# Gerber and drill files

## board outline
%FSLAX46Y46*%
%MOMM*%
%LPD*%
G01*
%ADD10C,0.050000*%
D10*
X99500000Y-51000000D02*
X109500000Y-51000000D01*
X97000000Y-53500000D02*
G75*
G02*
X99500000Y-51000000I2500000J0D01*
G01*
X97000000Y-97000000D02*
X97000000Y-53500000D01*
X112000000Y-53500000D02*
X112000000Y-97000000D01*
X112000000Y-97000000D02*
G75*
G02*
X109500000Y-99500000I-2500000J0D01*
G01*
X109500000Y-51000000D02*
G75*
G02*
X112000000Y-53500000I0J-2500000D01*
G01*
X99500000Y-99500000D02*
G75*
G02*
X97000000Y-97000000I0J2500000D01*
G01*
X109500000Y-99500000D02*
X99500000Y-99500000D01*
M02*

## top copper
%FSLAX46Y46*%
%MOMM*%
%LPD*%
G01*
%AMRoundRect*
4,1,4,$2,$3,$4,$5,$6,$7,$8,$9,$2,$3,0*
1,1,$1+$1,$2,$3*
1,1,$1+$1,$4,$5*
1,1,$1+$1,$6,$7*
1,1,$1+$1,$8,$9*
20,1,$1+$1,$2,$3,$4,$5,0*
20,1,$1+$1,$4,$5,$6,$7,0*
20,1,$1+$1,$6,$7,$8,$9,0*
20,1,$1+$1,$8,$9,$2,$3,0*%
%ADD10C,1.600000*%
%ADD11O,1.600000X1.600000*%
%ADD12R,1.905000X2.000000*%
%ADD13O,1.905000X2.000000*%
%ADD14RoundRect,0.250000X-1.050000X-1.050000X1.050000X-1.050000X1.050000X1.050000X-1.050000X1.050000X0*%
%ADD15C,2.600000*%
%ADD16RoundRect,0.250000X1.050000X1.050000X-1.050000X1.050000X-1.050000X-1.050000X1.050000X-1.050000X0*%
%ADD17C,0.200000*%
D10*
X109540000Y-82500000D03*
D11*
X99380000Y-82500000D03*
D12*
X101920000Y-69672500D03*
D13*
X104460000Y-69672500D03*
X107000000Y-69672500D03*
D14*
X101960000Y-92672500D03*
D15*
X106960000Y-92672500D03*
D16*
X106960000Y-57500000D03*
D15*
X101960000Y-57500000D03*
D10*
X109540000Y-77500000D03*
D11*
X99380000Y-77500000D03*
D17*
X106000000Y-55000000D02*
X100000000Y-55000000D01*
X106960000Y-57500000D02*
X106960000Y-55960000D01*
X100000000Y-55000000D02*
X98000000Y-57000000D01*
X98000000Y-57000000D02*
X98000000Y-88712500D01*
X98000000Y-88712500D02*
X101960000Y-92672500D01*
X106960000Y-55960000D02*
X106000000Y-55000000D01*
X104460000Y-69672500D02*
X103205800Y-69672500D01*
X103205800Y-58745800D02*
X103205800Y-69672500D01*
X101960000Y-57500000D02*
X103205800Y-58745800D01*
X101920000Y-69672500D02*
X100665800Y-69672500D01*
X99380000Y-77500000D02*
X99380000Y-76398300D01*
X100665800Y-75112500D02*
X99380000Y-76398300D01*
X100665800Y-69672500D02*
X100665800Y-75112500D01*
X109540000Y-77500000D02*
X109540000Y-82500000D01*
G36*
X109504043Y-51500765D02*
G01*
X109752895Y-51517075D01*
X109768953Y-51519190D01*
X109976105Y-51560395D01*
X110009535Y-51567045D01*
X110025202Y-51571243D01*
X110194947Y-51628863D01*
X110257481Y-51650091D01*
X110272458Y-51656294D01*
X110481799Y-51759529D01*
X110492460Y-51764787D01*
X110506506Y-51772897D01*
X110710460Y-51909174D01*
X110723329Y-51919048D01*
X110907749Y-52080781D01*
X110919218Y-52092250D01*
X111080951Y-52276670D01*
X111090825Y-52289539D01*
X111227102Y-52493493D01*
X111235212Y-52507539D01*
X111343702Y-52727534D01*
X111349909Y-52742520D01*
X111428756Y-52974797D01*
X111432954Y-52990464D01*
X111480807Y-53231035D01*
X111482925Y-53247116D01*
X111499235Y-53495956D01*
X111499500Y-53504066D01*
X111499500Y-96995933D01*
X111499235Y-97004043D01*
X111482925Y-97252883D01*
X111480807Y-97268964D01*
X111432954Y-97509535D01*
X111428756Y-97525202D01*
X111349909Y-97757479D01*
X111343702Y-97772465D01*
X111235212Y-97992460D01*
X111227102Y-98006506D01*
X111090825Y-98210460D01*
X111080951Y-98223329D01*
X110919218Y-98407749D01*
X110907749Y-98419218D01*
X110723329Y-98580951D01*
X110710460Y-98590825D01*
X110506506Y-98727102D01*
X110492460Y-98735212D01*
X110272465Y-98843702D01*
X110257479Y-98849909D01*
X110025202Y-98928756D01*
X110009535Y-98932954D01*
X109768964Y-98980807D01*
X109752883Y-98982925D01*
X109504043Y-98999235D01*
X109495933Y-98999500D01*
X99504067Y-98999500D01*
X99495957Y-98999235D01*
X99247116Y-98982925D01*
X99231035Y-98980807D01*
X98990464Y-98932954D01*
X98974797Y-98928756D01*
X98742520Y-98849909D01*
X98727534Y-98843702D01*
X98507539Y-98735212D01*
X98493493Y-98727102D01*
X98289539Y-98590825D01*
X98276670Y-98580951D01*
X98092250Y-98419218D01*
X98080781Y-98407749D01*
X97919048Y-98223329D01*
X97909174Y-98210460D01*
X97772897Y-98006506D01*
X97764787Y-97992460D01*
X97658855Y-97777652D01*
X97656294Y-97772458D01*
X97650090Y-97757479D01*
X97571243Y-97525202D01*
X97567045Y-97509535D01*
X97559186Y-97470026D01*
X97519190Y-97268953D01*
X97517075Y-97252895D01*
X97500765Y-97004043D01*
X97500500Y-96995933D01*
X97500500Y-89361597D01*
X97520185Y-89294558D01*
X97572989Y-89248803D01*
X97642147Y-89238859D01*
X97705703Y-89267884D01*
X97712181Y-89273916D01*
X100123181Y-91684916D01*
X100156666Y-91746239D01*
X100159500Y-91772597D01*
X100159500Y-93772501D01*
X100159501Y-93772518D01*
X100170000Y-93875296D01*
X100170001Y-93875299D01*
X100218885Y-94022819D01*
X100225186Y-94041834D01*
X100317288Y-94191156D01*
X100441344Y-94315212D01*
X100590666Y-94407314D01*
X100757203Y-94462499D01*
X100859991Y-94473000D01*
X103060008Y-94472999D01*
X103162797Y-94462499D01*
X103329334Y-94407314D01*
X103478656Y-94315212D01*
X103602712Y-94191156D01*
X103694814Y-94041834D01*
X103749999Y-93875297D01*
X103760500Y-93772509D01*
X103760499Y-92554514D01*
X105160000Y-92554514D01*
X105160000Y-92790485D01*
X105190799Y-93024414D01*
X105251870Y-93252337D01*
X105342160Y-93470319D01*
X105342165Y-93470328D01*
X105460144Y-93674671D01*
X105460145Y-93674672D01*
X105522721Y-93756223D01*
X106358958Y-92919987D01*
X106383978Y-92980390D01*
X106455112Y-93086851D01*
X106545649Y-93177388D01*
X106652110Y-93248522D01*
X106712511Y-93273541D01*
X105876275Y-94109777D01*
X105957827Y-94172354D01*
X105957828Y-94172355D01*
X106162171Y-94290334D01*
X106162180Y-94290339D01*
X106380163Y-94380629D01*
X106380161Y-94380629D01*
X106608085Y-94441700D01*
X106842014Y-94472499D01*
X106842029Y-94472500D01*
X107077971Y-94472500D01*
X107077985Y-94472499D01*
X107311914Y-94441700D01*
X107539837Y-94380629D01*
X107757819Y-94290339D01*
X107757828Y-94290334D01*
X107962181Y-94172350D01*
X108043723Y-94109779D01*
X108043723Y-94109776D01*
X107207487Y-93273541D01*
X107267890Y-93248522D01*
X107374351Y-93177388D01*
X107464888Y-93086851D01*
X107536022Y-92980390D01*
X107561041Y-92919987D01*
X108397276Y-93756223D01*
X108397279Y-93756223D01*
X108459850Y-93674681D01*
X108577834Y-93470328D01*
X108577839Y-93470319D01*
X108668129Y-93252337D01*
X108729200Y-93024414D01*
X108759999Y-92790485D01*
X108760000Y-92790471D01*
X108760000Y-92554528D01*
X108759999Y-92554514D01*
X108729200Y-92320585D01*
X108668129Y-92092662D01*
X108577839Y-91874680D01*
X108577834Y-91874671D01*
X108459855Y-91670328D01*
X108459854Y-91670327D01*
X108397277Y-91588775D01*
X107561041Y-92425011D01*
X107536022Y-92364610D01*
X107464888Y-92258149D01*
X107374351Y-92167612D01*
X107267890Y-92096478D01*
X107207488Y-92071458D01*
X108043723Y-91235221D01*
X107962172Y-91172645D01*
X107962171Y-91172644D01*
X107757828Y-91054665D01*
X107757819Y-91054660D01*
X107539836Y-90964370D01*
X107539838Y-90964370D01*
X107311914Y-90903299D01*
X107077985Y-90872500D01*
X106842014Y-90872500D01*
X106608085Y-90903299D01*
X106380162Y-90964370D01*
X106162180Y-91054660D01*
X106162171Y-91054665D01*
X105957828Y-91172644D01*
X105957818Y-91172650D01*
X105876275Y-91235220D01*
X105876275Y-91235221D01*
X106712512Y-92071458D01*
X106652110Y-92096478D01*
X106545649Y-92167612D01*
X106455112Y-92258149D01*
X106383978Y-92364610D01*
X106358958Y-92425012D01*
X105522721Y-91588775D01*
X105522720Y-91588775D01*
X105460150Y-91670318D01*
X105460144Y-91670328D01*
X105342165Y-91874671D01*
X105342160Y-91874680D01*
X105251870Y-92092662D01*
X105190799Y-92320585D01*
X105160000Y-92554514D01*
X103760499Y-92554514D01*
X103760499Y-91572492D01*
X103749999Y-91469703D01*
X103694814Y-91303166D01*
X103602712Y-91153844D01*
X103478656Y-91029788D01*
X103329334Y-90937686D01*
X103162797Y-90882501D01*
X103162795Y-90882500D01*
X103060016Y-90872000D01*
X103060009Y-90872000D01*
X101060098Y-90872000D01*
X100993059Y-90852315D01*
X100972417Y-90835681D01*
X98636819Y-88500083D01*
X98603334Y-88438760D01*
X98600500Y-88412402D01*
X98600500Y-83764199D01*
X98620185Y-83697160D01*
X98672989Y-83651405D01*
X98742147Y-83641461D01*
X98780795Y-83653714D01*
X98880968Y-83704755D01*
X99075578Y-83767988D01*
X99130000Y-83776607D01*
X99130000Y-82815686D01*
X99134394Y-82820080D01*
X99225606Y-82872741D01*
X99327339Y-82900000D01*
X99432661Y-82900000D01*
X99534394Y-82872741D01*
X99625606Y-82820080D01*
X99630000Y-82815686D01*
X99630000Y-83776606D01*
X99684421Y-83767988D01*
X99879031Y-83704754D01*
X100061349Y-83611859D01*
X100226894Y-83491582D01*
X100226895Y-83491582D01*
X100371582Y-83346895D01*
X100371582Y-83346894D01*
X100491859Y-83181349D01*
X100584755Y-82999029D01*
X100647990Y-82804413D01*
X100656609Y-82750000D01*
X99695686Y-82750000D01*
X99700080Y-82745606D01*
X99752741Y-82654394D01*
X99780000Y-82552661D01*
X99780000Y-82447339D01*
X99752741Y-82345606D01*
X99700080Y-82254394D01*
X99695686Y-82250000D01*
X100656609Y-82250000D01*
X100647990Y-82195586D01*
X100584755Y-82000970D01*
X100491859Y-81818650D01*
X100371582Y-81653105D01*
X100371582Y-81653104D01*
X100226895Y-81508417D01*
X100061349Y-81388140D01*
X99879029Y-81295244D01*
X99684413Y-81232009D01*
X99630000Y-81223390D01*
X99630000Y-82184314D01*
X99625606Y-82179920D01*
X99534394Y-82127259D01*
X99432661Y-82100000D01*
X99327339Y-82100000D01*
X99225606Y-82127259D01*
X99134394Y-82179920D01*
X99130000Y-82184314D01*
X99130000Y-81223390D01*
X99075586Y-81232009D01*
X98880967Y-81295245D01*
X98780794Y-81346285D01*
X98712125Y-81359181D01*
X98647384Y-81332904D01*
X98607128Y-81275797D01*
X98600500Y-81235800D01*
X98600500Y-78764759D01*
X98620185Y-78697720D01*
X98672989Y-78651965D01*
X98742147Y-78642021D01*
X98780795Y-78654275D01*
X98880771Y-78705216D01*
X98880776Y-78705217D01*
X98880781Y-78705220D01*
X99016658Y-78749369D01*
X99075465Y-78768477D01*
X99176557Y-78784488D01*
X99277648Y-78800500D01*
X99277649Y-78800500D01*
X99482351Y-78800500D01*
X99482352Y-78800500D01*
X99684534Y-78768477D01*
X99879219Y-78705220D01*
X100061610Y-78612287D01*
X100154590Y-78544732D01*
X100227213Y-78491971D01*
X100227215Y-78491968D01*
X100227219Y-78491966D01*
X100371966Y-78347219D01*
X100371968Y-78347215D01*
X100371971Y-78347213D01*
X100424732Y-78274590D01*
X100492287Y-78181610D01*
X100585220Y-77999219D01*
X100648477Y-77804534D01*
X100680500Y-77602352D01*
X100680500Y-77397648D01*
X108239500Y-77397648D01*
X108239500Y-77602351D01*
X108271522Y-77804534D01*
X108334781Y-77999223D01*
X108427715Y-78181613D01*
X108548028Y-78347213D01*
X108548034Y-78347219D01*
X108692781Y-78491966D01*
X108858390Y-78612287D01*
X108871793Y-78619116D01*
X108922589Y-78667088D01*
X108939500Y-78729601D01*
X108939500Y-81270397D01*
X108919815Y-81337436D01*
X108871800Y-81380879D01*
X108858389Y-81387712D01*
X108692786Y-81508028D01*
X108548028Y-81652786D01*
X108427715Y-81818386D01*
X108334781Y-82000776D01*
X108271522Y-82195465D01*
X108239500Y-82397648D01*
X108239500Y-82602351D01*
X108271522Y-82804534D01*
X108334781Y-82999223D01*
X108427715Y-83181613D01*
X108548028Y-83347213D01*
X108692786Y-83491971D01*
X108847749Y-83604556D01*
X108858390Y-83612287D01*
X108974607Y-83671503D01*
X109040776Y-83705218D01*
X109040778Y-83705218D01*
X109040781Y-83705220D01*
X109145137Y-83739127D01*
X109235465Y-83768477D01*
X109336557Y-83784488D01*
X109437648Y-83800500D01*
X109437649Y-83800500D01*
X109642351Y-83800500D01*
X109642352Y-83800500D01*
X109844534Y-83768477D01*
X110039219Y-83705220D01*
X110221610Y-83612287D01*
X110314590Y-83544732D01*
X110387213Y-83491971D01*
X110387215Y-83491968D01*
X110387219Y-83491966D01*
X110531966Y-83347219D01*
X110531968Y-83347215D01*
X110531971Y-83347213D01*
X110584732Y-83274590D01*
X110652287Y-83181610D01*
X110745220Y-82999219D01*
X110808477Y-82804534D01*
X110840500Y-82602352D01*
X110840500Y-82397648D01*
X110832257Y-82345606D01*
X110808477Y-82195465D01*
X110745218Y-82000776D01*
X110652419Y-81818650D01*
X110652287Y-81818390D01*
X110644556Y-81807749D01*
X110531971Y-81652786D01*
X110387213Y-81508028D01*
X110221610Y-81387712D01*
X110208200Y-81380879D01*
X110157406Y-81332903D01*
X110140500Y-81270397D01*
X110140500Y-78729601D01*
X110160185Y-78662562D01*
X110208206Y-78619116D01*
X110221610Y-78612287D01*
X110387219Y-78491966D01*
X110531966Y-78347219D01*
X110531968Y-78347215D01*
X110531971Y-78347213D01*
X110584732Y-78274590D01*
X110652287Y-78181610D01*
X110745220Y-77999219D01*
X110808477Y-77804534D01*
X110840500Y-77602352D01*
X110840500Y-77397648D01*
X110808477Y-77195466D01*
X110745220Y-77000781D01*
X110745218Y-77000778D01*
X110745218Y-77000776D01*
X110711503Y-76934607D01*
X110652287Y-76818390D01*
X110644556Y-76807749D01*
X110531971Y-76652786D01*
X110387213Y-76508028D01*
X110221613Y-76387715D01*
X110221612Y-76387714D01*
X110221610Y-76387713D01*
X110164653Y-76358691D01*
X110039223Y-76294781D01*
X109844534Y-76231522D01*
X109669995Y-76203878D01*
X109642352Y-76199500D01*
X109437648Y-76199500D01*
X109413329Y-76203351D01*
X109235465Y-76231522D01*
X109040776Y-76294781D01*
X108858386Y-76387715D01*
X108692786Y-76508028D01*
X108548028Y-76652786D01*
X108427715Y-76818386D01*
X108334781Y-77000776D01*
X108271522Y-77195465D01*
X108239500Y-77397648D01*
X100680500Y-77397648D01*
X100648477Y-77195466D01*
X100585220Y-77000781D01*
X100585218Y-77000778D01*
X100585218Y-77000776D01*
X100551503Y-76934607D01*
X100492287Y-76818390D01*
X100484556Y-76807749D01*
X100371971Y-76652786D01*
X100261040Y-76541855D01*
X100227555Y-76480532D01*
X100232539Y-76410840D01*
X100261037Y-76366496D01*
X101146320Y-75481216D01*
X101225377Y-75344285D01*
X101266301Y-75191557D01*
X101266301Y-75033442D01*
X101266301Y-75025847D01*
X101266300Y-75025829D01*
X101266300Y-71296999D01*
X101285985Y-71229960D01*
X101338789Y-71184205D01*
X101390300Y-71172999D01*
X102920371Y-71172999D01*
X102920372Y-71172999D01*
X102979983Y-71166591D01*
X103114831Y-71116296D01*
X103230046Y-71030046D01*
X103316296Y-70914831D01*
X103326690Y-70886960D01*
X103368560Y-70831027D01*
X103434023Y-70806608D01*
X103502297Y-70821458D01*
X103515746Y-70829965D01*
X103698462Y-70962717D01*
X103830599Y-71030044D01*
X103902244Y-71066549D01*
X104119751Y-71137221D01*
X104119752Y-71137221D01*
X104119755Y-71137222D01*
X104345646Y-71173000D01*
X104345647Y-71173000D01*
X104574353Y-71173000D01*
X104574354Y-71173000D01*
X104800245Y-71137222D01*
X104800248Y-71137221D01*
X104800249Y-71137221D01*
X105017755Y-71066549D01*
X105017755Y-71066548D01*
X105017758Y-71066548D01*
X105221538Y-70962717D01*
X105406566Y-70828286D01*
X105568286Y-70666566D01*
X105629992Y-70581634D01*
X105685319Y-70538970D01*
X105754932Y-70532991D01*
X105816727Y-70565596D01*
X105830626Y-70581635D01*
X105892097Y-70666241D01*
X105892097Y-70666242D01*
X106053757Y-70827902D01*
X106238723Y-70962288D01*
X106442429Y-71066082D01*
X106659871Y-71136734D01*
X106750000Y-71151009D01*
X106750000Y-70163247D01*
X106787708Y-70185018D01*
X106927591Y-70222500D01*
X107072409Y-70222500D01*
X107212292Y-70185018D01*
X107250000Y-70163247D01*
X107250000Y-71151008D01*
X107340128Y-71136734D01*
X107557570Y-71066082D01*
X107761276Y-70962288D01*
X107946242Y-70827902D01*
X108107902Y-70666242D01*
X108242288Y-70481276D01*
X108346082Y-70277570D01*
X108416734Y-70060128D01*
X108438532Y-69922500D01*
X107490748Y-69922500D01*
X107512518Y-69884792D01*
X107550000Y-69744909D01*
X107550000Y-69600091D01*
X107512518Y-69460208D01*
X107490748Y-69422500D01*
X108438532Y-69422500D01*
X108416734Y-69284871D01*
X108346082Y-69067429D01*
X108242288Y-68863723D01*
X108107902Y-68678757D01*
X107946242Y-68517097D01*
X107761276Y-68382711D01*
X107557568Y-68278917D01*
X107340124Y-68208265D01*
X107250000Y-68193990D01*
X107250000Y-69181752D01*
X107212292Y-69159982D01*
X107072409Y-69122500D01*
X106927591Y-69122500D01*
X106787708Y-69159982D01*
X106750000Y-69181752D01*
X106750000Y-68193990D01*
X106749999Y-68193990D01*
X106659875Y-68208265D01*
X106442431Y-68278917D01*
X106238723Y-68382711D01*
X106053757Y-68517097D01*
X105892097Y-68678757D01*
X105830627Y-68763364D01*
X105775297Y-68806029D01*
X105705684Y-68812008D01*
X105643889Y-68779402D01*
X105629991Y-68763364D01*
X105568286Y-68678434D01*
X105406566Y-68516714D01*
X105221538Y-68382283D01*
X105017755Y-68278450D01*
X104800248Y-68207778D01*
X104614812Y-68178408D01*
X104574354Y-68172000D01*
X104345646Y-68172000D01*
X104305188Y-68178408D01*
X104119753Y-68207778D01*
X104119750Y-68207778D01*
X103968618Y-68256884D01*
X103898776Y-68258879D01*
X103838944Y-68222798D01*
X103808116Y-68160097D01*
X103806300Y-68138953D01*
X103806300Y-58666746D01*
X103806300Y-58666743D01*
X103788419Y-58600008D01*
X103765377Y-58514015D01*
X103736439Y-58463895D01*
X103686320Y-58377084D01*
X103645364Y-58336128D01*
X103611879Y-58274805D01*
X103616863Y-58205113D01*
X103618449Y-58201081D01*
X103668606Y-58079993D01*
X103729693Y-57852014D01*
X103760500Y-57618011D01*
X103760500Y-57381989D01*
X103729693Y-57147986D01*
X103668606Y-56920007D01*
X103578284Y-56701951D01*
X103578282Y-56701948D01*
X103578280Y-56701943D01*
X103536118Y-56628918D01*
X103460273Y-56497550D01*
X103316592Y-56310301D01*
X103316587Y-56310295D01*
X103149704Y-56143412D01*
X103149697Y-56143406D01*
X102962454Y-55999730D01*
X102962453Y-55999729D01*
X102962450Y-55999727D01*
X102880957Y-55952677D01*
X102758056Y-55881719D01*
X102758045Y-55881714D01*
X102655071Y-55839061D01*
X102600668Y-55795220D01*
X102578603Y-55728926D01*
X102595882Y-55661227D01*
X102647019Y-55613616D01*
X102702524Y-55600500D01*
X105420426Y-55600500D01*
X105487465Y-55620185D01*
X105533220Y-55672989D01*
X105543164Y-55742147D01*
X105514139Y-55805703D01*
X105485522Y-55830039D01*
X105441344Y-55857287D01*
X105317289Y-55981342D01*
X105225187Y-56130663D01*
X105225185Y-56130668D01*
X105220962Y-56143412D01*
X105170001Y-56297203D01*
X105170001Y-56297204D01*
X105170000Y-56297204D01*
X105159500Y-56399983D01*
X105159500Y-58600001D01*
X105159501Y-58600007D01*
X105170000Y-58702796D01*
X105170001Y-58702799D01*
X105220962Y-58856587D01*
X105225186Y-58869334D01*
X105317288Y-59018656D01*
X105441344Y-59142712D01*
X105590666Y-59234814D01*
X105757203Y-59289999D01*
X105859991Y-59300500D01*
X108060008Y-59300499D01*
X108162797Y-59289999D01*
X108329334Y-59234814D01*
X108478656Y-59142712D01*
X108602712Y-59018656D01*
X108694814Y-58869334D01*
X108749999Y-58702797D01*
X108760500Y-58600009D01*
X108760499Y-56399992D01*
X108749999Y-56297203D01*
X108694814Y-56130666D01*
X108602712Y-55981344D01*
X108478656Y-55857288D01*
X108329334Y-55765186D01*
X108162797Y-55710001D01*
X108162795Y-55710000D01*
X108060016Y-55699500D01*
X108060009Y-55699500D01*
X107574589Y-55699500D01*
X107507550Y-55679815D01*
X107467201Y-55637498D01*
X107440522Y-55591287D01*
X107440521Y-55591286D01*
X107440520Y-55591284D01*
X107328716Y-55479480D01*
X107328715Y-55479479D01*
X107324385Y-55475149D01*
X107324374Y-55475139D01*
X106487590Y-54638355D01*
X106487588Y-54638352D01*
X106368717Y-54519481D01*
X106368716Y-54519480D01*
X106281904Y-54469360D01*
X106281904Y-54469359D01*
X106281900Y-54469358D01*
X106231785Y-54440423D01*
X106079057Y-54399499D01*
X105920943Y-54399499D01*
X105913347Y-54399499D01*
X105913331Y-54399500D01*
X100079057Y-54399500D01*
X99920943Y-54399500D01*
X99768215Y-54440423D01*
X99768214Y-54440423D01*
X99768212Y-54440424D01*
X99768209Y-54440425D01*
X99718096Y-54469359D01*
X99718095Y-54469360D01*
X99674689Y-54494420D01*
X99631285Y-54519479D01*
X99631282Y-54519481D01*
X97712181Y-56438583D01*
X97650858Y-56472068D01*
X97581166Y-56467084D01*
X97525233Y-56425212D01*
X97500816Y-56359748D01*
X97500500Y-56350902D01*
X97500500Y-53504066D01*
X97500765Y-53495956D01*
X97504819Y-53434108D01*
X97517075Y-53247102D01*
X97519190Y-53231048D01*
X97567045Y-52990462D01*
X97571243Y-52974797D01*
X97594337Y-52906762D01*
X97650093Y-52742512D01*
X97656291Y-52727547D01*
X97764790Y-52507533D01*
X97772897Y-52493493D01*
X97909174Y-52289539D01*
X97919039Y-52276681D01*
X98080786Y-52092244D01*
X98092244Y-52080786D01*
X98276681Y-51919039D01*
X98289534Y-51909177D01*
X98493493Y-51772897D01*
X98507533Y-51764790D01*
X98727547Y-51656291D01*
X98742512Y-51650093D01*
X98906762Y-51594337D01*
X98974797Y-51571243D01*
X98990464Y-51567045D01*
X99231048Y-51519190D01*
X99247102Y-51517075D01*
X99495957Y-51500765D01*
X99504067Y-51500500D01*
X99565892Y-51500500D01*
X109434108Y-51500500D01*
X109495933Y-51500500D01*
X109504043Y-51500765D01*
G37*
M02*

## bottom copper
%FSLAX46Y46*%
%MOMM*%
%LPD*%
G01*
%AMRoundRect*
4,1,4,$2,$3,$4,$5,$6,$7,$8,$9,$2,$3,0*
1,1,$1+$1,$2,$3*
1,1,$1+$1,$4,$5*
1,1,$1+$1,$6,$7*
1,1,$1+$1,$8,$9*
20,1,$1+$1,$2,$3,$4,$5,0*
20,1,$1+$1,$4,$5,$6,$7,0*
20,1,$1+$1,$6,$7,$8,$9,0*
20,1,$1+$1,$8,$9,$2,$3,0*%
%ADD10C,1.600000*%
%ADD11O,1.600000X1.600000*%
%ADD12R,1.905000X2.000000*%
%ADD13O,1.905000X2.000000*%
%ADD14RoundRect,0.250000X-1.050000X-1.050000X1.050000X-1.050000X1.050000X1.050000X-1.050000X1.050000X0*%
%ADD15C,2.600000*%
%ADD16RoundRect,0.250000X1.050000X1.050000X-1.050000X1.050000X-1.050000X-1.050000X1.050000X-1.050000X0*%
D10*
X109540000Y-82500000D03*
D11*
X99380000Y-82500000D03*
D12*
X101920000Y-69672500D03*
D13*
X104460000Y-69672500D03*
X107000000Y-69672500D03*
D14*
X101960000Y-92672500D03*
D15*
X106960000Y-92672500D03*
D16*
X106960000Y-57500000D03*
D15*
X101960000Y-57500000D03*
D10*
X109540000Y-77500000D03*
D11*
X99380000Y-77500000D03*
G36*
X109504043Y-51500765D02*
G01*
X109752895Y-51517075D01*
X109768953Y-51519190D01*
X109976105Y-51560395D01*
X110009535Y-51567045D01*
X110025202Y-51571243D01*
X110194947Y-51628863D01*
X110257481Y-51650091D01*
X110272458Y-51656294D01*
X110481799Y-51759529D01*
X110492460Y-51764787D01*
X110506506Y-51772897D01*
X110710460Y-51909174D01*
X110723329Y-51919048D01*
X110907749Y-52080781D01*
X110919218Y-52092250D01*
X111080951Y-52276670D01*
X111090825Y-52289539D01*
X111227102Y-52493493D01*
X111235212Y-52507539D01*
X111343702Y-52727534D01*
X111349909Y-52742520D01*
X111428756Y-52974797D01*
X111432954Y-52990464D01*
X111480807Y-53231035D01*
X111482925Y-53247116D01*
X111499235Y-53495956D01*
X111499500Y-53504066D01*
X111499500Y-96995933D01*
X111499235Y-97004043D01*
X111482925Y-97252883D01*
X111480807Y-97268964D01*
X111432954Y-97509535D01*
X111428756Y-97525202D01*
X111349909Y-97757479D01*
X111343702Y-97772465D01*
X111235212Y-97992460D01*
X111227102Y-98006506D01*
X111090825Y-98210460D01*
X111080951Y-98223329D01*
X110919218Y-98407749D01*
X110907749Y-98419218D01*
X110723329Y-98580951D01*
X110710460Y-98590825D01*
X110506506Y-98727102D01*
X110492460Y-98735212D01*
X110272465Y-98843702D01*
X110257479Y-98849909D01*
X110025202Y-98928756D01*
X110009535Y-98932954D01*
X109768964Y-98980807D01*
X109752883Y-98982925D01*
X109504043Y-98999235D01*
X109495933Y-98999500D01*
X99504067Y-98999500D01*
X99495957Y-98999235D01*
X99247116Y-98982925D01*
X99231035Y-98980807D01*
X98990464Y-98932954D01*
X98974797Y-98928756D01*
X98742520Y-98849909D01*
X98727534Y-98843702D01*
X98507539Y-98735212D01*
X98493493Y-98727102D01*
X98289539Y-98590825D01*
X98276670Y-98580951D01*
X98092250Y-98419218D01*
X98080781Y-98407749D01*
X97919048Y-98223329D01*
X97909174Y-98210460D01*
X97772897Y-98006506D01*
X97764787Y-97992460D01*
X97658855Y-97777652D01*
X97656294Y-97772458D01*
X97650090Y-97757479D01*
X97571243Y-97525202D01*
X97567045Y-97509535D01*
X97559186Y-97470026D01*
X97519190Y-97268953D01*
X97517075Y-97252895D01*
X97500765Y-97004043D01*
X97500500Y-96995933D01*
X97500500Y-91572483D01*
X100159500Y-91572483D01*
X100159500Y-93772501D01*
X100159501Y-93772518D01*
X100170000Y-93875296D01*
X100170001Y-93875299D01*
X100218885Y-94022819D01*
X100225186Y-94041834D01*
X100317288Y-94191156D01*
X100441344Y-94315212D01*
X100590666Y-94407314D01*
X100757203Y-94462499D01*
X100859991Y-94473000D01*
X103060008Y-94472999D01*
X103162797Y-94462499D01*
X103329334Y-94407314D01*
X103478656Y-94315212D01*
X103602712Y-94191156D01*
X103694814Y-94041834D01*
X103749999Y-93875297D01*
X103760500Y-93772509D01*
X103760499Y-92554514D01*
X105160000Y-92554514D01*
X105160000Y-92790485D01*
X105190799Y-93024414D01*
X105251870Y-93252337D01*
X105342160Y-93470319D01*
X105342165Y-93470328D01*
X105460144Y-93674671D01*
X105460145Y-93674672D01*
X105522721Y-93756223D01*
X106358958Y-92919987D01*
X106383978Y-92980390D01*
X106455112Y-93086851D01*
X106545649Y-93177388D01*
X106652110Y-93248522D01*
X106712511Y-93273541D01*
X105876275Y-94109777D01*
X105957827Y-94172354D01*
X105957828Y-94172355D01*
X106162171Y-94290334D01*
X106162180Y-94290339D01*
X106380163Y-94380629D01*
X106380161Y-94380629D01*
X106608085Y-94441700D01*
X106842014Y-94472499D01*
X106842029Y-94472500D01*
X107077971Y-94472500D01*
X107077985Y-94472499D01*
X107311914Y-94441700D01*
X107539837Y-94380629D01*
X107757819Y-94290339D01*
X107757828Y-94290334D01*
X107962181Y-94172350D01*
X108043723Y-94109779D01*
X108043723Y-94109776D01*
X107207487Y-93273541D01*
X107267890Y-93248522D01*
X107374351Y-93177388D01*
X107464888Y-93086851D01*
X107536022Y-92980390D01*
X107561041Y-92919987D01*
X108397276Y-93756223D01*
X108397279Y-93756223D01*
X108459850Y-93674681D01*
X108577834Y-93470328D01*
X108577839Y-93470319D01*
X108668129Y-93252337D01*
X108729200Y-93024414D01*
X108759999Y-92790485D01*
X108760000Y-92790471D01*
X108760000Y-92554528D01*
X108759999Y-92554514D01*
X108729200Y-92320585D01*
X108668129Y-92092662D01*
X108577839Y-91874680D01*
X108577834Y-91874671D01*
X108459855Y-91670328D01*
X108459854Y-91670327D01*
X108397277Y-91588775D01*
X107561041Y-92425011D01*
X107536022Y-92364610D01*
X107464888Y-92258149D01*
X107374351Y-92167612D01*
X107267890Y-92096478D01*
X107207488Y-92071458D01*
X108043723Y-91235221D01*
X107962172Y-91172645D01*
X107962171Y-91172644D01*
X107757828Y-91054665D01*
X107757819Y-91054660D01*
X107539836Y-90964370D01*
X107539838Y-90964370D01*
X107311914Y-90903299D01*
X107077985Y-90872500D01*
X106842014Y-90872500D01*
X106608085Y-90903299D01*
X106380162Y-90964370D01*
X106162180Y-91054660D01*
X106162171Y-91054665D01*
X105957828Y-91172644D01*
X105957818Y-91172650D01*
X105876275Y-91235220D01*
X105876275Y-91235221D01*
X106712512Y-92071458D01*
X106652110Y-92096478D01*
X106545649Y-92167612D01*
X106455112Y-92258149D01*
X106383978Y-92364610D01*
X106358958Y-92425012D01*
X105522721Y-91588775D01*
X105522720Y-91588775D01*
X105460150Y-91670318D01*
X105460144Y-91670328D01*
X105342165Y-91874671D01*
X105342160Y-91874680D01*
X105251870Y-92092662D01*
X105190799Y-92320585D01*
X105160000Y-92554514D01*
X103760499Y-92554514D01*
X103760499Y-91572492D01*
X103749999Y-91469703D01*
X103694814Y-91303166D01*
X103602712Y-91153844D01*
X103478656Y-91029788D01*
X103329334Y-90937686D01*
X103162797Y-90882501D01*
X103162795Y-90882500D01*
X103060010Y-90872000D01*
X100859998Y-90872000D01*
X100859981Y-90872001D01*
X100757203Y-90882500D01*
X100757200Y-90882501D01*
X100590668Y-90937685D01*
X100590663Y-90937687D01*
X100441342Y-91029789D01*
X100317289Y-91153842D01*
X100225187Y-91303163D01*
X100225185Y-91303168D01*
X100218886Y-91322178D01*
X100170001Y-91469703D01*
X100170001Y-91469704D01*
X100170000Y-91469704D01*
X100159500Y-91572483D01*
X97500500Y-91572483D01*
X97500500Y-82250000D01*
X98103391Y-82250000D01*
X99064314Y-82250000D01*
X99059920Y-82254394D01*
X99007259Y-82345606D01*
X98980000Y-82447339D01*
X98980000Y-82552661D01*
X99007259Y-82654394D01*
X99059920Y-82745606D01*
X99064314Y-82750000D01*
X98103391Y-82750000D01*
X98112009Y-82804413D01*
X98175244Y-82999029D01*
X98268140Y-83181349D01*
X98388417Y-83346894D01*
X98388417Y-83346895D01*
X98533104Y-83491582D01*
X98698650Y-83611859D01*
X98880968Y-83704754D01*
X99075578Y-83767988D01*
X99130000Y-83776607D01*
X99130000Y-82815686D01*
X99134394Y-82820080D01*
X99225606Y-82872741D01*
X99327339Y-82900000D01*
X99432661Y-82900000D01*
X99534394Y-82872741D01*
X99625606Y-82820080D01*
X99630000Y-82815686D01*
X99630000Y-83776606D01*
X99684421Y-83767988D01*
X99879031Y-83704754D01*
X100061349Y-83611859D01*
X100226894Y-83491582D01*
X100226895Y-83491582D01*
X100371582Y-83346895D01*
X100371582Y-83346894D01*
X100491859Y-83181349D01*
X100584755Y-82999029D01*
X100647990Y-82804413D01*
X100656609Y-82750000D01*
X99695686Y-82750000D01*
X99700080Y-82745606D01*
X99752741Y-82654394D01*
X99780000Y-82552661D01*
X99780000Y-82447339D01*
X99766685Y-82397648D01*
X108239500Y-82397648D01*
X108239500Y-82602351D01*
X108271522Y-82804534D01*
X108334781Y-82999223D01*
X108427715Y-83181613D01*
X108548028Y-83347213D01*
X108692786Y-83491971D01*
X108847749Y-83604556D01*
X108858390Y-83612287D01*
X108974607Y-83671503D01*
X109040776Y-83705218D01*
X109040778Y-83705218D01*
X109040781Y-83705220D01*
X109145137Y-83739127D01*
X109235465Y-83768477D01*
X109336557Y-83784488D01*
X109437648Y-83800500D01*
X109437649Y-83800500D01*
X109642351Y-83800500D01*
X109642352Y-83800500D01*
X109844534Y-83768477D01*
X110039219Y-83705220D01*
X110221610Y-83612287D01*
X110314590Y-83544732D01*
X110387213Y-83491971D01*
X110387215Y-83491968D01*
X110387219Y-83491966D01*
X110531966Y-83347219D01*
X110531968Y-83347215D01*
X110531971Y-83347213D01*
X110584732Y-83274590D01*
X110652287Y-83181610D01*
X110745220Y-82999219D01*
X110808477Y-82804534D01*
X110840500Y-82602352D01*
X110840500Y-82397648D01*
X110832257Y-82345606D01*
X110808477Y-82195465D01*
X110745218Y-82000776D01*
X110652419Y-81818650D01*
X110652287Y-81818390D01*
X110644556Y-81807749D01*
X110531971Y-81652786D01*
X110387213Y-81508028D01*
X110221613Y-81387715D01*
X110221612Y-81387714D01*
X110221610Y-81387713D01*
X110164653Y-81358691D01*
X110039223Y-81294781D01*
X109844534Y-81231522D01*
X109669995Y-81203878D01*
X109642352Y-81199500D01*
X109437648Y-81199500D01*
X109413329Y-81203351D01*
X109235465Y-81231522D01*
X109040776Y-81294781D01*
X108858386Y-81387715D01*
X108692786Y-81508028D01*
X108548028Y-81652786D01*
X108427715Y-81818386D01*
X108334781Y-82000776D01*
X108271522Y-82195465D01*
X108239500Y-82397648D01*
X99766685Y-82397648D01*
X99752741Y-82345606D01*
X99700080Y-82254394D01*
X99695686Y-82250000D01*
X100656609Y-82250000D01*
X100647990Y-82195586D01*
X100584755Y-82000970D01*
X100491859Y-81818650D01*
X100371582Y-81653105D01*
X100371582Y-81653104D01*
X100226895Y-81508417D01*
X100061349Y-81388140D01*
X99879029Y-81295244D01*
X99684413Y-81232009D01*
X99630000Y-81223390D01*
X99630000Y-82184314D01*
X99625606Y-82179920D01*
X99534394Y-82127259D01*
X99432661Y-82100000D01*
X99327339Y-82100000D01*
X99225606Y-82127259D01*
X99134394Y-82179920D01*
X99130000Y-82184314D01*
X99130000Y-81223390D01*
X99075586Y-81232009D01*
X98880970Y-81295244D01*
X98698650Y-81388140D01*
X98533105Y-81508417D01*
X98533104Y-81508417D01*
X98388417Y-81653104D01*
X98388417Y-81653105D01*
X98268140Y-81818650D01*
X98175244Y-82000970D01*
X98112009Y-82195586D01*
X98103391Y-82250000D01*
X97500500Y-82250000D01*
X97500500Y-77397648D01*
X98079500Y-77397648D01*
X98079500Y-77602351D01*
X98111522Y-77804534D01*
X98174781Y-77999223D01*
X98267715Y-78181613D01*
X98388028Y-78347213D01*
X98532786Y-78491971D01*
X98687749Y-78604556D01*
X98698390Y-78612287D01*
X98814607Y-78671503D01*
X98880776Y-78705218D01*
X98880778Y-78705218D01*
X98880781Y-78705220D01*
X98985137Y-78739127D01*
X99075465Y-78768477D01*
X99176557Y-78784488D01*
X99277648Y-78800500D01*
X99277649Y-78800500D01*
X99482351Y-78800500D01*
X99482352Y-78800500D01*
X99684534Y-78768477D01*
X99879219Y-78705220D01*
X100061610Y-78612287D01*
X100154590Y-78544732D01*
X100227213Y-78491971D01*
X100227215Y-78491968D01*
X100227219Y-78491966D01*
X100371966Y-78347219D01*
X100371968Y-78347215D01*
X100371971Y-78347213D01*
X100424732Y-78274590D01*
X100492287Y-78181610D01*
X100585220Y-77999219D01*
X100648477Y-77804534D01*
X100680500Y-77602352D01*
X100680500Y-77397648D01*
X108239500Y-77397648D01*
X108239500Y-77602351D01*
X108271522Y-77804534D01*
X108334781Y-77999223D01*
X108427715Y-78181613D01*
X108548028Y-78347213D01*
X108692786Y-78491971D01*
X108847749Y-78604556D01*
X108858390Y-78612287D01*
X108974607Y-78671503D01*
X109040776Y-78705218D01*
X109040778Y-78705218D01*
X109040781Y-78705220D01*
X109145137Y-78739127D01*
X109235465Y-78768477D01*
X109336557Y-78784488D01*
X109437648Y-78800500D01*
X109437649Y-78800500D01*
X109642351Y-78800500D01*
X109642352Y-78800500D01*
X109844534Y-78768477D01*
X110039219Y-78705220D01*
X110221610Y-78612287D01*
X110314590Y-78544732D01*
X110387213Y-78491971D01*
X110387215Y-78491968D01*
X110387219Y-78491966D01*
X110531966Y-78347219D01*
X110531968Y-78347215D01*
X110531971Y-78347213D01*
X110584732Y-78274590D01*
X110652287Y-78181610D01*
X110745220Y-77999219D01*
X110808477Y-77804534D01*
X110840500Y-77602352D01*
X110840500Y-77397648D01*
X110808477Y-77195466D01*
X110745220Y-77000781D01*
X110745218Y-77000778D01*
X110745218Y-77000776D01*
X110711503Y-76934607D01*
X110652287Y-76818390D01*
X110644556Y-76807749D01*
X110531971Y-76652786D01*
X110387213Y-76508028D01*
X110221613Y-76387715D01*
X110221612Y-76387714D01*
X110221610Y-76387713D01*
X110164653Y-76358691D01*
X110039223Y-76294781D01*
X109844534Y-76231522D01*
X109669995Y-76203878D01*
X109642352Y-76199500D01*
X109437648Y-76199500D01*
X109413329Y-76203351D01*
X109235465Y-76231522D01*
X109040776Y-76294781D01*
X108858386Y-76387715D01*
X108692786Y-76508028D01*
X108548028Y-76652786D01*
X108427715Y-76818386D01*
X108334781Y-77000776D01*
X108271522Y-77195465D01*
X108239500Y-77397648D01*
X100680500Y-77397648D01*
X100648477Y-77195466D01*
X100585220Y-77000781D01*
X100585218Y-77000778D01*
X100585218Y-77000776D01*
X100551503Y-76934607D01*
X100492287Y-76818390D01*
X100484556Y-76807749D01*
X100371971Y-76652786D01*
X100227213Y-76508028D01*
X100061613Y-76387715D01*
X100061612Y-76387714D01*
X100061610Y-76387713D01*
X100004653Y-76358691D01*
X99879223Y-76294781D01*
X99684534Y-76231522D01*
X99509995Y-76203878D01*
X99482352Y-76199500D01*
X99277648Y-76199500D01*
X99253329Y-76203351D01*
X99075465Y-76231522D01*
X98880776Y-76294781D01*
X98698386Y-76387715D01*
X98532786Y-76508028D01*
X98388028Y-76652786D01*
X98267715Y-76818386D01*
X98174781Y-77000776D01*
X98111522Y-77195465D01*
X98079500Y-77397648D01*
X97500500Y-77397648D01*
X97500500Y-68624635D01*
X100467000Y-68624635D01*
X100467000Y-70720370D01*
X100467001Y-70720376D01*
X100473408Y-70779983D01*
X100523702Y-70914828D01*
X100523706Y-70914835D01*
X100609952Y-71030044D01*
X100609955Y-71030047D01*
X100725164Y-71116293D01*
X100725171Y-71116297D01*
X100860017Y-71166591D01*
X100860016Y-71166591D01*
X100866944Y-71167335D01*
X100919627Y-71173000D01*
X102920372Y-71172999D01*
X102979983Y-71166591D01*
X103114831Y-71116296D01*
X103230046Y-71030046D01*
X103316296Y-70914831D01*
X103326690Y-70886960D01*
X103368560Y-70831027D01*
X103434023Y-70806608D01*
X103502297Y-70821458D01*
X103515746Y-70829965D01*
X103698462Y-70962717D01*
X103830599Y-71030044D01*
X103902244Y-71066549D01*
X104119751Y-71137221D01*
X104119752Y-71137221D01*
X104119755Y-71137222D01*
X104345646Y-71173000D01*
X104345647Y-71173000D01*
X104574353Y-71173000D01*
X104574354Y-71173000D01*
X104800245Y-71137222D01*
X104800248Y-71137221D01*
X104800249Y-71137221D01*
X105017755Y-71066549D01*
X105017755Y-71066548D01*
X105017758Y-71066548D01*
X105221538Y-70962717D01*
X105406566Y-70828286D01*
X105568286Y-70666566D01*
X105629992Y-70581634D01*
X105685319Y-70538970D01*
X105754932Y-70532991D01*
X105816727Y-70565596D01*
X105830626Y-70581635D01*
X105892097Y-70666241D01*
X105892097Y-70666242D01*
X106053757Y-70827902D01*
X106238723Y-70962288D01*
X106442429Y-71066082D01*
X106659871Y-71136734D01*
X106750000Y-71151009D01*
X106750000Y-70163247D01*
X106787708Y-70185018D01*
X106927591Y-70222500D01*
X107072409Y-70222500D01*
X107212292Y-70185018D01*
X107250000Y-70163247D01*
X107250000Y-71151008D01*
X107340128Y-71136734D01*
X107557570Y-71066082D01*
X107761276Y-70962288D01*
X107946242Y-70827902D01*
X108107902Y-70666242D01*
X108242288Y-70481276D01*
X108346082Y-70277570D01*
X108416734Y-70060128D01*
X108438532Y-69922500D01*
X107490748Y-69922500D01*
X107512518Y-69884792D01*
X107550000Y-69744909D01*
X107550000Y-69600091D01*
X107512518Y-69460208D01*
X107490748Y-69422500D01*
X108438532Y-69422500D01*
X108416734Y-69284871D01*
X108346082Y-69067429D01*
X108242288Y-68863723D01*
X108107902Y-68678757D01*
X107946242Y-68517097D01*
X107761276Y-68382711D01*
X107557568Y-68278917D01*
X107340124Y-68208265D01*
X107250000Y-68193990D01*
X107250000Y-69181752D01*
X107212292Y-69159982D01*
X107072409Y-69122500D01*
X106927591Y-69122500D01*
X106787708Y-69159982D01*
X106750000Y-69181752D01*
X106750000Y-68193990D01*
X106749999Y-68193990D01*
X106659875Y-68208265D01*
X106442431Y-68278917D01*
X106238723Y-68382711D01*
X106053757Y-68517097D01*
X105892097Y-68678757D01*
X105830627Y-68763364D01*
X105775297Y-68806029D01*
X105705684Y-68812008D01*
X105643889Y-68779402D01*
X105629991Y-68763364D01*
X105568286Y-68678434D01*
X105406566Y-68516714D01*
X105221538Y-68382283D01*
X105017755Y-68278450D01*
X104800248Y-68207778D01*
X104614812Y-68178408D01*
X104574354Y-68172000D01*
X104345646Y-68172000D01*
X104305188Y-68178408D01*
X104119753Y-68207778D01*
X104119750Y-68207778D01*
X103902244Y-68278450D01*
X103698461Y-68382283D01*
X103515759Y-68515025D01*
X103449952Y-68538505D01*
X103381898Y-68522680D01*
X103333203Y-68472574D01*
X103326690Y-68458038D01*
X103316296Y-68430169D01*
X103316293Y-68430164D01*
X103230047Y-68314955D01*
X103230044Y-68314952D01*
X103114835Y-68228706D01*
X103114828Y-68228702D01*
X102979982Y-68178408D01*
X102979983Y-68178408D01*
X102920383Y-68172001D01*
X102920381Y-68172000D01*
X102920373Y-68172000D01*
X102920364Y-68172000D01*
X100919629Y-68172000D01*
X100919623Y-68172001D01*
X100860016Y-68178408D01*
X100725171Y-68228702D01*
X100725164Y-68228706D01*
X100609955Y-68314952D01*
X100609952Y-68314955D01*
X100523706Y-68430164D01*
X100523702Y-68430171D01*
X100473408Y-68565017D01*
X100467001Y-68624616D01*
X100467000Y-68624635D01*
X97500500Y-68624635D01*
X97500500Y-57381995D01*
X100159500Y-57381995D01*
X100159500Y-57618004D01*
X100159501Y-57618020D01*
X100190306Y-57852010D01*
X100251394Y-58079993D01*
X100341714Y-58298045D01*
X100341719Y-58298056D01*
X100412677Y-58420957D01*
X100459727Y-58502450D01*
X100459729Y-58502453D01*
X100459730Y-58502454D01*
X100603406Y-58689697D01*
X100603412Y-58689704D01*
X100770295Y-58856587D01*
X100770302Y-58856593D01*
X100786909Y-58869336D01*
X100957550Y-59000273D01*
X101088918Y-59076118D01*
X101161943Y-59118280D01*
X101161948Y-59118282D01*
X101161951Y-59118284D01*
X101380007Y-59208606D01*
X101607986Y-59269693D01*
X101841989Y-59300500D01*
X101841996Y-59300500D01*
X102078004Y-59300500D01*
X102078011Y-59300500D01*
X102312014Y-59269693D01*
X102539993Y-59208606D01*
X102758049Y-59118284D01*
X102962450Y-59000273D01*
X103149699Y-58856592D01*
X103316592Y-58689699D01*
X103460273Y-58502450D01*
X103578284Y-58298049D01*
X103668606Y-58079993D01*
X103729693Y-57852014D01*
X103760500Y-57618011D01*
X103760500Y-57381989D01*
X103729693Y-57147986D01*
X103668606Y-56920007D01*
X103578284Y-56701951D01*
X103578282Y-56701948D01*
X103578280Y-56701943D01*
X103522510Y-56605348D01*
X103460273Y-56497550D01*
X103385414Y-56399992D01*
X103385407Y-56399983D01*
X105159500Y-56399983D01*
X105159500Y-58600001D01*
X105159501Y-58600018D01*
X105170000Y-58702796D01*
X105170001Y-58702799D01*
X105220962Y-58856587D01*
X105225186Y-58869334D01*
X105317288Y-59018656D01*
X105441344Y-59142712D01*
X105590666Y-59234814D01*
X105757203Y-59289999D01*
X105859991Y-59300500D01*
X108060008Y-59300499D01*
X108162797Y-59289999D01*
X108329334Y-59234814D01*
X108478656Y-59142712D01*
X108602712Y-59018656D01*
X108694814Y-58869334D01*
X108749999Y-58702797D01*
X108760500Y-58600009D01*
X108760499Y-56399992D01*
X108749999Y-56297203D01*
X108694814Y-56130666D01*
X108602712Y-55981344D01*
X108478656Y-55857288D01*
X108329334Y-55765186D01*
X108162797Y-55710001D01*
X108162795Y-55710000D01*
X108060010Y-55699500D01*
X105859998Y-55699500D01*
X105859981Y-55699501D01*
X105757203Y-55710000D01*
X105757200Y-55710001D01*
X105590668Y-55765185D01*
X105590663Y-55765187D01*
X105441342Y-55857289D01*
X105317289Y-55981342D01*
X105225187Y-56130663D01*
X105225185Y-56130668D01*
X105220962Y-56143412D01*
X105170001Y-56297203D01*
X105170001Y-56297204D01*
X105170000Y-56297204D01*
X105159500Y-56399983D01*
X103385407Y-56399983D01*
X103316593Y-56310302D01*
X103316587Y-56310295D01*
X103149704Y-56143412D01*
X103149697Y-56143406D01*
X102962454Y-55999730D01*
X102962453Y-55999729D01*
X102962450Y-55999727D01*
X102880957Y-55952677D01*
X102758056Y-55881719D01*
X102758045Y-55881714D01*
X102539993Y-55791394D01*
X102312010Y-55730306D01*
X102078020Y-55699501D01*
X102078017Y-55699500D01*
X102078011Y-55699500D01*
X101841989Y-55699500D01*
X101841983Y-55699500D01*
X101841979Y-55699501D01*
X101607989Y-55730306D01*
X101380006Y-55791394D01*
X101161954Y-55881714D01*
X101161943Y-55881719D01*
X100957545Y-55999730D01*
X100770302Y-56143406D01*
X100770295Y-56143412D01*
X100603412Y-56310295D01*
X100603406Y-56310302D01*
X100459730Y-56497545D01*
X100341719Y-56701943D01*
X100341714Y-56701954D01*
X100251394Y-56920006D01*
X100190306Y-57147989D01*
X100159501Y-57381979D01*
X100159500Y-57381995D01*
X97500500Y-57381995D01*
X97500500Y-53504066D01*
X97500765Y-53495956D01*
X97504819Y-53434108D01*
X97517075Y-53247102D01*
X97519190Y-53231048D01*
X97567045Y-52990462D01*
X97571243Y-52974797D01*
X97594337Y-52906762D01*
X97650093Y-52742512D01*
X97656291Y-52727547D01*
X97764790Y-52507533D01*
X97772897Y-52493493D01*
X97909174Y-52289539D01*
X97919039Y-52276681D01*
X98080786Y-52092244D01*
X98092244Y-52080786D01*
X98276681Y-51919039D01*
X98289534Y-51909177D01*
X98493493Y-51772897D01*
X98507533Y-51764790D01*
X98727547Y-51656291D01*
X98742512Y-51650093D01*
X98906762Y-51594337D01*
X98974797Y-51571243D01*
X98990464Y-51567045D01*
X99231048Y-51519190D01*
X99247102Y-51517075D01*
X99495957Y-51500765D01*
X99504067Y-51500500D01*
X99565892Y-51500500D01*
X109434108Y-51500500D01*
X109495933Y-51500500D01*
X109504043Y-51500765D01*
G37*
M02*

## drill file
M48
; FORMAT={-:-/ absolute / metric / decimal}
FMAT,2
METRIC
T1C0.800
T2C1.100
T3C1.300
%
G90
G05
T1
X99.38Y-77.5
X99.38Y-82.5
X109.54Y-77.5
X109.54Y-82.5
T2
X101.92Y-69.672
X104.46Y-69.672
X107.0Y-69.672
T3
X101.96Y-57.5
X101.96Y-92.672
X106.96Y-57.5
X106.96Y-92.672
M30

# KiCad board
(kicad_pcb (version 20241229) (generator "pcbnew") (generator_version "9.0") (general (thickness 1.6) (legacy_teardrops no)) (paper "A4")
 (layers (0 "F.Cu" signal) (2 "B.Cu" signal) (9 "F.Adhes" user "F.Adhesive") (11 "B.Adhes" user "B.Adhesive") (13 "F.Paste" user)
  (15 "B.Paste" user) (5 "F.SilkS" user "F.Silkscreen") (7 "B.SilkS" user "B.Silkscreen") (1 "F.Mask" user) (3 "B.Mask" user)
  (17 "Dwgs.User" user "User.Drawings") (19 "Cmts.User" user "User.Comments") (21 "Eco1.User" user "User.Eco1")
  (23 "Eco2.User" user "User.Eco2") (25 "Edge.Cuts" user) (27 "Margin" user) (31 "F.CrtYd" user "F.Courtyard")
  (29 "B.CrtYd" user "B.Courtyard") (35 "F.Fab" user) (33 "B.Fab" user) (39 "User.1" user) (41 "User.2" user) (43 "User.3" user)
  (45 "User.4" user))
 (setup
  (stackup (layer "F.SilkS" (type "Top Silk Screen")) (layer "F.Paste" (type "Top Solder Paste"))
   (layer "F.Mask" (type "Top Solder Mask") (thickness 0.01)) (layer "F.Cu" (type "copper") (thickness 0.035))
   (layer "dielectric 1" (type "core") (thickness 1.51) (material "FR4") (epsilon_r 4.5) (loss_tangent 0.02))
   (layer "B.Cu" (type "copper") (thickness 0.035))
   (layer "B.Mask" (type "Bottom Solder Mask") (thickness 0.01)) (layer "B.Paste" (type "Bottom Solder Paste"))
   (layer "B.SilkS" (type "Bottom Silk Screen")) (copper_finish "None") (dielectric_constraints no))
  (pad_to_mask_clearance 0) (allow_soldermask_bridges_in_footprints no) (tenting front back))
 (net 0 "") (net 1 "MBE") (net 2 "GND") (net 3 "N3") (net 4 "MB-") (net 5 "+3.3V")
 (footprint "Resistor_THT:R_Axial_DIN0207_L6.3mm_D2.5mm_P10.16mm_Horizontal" (layer "F.Cu") (at 109.54 82.5 180)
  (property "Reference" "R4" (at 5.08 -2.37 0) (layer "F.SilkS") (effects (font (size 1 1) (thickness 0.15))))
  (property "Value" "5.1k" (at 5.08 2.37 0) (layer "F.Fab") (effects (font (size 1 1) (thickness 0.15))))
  (pad "1" thru_hole circle (at 0 0 180) (size 1.6 1.6) (drill 0.8) (layers "*.Cu" "*.Mask") (remove_unused_layers no) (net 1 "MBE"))
  (pad "2" thru_hole oval (at 10.16 0 180) (size 1.6 1.6) (drill 0.8) (layers "*.Cu" "*.Mask") (remove_unused_layers no) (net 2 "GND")))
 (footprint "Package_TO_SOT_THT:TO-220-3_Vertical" (layer "F.Cu") (at 101.92 69.6725)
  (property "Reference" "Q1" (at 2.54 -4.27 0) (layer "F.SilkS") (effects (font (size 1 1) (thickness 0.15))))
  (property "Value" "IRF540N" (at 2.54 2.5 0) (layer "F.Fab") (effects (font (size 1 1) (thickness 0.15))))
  (pad "1" thru_hole rect (at 0 0) (size 1.905 2) (drill 1.1) (layers "*.Cu" "*.Mask") (remove_unused_layers no) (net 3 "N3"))
  (pad "2" thru_hole oval (at 2.54 0) (size 1.905 2) (drill 1.1) (layers "*.Cu" "*.Mask") (remove_unused_layers no) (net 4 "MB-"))
  (pad "3" thru_hole oval (at 5.08 0) (size 1.905 2) (drill 1.1) (layers "*.Cu" "*.Mask") (remove_unused_layers no) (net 2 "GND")))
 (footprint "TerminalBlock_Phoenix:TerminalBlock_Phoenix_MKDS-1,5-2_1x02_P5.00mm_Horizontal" (layer "F.Cu") (at 101.96 92.6725)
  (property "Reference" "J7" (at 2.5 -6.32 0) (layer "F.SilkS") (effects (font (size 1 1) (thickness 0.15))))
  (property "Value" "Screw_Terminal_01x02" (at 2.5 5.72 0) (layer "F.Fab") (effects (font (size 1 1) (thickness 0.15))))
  (pad "1" thru_hole roundrect (at 0 0) (size 2.6 2.6) (drill 1.3) (layers "*.Cu" "*.Mask") (remove_unused_layers no)
   (roundrect_rratio 0.096154) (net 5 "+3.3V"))
  (pad "2" thru_hole circle (at 5 0) (size 2.6 2.6) (drill 1.3) (layers "*.Cu" "*.Mask") (remove_unused_layers no) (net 2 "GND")))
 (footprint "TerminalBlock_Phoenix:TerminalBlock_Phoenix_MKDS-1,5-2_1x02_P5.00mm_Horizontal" (layer "F.Cu") (at 106.96 57.5 180)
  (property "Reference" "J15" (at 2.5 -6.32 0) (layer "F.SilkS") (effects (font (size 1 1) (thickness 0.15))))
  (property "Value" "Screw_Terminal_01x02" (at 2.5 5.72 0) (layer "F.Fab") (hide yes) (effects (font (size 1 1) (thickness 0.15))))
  (pad "1" thru_hole roundrect (at 0 0 180) (size 2.6 2.6) (drill 1.3) (layers "*.Cu" "*.Mask") (remove_unused_layers no)
   (roundrect_rratio 0.096154) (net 5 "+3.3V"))
  (pad "2" thru_hole circle (at 5 0 180) (size 2.6 2.6) (drill 1.3) (layers "*.Cu" "*.Mask") (remove_unused_layers no) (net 4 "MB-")))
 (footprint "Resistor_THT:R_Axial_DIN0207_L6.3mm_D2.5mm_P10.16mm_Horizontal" (layer "F.Cu") (at 109.54 77.5 180)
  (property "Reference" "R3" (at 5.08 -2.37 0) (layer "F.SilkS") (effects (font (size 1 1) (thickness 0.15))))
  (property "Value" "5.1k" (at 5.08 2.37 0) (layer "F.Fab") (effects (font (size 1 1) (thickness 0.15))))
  (pad "1" thru_hole circle (at 0 0 180) (size 1.6 1.6) (drill 0.8) (layers "*.Cu" "*.Mask") (remove_unused_layers no) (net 1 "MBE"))
  (pad "2" thru_hole oval (at 10.16 0 180) (size 1.6 1.6) (drill 0.8) (layers "*.Cu" "*.Mask") (remove_unused_layers no) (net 3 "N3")))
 (gr_line (start 99.5 51) (end 109.5 51) (stroke (width 0.05) (type default)) (layer "Edge.Cuts"))
 (gr_arc (start 97 53.5) (mid 97.732233 51.732233) (end 99.5 51) (stroke (width 0.05) (type default)) (layer "Edge.Cuts"))
 (gr_line (start 97 97) (end 97 53.5) (stroke (width 0.05) (type default)) (layer "Edge.Cuts"))
 (gr_line (start 112 53.5) (end 112 97) (stroke (width 0.05) (type default)) (layer "Edge.Cuts"))
 (gr_arc (start 112 97) (mid 111.267767 98.767767) (end 109.5 99.5) (stroke (width 0.05) (type default)) (layer "Edge.Cuts"))
 (gr_arc (start 109.5 51) (mid 111.267767 51.732233) (end 112 53.5) (stroke (width 0.05) (type default)) (layer "Edge.Cuts"))
 (gr_arc (start 99.5 99.5) (mid 97.732233 98.767767) (end 97 97) (stroke (width 0.05) (type default)) (layer "Edge.Cuts"))
 (gr_line (start 109.5 99.5) (end 99.5 99.5) (stroke (width 0.05) (type default)) (layer "Edge.Cuts"))
 (segment (start 106 55) (end 100 55) (width 0.2) (layer "F.Cu") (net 5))
 (segment (start 106.96 57.5) (end 106.96 55.96) (width 0.2) (layer "F.Cu") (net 5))
 (segment (start 100 55) (end 98 57) (width 0.2) (layer "F.Cu") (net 5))
 (segment (start 98 57) (end 98 88.7125) (width 0.2) (layer "F.Cu") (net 5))
 (segment (start 98 88.7125) (end 101.96 92.6725) (width 0.2) (layer "F.Cu") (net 5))
 (segment (start 106.96 55.96) (end 106 55) (width 0.2) (layer "F.Cu") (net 5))
 (segment (start 104.46 69.6725) (end 103.2058 69.6725) (width 0.2) (layer "F.Cu") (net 4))
 (segment (start 103.2058 58.7458) (end 103.2058 69.6725) (width 0.2) (layer "F.Cu") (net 4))
 (segment (start 101.96 57.5) (end 103.2058 58.7458) (width 0.2) (layer "F.Cu") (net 4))
 (segment (start 101.92 69.6725) (end 100.6658 69.6725) (width 0.2) (layer "F.Cu") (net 3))
 (segment (start 99.38 77.5) (end 99.38 76.3983) (width 0.2) (layer "F.Cu") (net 3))
 (segment (start 100.6658 75.1125) (end 99.38 76.3983) (width 0.2) (layer "F.Cu") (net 3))
 (segment (start 100.6658 69.6725) (end 100.6658 75.1125) (width 0.2) (layer "F.Cu") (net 3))
 (segment (start 109.54 77.5) (end 109.54 82.5) (width 0.2) (layer "F.Cu") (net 1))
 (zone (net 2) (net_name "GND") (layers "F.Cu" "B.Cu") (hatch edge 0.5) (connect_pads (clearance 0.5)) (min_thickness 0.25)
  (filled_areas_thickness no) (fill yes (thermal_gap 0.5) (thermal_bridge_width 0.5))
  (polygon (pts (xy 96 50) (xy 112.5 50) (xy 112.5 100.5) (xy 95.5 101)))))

